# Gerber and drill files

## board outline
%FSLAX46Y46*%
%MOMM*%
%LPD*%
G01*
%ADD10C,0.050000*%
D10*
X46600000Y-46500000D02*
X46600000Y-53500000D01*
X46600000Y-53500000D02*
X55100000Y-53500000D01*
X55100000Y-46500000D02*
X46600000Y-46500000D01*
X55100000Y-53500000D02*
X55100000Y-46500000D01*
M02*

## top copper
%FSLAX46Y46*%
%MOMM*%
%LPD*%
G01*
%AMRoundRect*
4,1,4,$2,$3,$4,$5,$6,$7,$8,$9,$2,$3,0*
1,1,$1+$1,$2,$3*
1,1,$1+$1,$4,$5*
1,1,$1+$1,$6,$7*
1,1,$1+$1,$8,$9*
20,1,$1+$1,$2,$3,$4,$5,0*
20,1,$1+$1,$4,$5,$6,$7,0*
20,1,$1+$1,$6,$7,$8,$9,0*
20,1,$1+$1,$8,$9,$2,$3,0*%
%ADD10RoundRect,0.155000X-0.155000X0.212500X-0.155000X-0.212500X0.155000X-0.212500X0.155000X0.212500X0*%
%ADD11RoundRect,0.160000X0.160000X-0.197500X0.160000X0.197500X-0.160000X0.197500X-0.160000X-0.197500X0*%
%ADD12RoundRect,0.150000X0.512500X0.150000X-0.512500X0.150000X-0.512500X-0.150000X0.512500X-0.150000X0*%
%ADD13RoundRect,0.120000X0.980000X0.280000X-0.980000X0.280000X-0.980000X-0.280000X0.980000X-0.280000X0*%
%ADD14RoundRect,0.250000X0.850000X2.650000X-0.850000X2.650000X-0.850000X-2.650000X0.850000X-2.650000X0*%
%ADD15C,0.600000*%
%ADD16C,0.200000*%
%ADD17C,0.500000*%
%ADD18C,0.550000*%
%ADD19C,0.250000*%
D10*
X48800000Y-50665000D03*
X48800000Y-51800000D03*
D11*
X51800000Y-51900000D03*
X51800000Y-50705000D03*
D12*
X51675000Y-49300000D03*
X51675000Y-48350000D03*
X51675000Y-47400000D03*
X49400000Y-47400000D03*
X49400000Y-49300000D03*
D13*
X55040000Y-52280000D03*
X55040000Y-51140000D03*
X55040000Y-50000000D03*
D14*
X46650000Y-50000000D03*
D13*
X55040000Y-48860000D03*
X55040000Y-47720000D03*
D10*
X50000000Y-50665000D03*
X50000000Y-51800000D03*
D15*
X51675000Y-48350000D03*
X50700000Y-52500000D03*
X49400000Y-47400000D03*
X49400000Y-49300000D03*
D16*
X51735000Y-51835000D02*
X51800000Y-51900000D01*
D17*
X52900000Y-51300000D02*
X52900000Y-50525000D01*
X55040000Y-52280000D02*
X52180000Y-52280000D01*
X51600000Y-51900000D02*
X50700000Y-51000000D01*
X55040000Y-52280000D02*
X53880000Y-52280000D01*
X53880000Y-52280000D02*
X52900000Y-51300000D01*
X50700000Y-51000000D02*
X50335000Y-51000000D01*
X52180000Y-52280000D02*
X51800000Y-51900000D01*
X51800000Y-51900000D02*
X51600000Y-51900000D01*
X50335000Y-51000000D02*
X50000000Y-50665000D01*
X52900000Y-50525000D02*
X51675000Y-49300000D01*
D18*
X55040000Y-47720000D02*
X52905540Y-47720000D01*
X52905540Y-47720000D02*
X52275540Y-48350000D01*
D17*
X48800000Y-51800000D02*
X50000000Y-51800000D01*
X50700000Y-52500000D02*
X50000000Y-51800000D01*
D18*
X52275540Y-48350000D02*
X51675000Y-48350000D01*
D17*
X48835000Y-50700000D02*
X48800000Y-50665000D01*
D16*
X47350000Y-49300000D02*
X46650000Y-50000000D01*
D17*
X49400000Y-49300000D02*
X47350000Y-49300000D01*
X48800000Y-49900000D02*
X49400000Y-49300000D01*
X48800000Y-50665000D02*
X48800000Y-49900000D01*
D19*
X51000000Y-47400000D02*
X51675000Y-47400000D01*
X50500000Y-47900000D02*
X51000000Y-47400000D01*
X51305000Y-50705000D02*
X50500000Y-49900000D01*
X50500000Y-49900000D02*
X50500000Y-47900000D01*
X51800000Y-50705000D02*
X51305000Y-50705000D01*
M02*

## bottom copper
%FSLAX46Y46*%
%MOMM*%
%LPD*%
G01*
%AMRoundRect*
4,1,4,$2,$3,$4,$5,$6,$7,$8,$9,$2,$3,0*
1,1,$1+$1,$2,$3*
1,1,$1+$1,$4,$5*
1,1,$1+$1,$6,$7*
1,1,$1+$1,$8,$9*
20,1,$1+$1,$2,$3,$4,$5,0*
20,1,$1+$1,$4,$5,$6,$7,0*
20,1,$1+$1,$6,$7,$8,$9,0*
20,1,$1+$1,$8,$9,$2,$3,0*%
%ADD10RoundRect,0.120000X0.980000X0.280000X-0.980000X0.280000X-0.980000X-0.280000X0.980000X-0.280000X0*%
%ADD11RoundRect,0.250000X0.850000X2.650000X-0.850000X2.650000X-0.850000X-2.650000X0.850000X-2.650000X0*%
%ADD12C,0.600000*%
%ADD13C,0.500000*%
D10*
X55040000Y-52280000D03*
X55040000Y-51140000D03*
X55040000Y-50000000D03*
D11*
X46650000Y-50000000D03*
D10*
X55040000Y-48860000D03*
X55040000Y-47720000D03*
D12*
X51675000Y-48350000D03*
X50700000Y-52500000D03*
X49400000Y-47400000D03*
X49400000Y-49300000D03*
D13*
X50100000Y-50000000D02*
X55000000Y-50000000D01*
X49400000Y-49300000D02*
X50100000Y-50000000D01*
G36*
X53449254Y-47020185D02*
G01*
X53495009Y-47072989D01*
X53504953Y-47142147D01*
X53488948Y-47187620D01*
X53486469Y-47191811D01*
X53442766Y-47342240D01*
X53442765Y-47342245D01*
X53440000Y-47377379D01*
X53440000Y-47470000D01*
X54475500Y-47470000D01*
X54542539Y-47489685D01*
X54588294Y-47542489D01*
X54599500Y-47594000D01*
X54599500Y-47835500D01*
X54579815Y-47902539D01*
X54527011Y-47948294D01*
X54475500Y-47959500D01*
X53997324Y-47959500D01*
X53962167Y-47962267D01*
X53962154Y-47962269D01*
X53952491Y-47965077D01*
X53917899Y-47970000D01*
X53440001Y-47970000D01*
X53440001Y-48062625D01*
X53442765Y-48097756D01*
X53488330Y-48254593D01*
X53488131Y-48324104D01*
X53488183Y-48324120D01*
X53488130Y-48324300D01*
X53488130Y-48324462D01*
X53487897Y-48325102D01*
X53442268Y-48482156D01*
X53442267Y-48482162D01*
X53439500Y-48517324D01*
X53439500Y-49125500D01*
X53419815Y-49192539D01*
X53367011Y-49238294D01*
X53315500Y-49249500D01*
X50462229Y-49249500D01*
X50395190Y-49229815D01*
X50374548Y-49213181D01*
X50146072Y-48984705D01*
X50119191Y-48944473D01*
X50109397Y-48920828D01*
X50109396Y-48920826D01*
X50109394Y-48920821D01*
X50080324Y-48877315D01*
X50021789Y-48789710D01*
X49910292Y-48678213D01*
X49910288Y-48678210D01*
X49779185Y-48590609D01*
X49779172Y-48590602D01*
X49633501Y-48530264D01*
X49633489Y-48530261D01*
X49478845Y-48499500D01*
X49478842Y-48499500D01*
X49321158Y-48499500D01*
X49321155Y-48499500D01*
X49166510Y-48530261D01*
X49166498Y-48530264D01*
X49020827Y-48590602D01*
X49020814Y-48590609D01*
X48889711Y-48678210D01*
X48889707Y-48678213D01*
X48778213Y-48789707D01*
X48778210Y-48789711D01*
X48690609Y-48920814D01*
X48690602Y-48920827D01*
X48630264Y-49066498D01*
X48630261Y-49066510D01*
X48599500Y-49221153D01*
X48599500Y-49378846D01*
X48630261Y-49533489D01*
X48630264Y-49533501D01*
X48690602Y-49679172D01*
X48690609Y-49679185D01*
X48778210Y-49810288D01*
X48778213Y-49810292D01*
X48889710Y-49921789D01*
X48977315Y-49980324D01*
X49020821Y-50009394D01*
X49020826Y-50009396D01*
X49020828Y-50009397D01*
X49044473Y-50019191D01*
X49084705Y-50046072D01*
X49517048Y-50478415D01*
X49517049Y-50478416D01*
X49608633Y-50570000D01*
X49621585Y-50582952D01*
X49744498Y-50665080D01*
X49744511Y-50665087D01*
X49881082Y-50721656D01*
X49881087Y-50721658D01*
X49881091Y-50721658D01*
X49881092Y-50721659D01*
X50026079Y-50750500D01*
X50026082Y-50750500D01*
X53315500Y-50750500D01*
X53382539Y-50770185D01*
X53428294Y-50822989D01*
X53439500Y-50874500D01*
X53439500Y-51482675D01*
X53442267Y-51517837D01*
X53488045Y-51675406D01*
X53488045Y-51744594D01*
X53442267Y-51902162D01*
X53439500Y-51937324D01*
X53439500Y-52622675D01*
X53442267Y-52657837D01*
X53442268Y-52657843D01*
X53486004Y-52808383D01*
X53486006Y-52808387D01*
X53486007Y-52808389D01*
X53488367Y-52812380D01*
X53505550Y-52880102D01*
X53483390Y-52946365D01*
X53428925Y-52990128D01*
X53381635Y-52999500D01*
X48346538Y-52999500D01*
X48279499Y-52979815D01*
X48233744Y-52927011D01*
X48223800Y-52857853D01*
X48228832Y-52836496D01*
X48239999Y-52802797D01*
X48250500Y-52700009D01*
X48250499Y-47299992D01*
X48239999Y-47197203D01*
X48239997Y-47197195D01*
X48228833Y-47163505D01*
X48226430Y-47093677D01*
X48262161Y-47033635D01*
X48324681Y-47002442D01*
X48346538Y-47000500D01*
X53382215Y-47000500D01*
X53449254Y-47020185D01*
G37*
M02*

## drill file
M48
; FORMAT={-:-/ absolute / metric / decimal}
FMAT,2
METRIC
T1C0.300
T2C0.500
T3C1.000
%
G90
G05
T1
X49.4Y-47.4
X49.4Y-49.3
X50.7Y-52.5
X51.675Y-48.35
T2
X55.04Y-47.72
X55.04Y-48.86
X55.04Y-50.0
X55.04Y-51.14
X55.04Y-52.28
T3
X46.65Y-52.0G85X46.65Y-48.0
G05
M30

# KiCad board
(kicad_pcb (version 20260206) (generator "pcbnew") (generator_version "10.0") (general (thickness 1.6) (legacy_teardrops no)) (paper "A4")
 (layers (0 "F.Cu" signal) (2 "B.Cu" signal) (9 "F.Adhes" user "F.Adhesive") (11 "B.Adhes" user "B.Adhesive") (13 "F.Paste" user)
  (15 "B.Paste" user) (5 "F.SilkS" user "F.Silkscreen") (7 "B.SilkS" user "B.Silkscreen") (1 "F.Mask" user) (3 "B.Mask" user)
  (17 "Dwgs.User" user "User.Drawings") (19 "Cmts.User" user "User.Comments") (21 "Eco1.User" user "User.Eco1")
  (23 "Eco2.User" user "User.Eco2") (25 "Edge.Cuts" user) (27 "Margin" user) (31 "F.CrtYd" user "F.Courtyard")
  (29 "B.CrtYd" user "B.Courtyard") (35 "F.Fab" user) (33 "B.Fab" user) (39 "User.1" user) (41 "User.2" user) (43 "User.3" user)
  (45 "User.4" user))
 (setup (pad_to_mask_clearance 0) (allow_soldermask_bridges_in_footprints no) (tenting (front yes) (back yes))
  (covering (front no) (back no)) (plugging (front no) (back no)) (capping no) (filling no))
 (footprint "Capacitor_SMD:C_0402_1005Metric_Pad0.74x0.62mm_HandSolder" (layer "F.Cu") (at 48.8 51.2325 -90)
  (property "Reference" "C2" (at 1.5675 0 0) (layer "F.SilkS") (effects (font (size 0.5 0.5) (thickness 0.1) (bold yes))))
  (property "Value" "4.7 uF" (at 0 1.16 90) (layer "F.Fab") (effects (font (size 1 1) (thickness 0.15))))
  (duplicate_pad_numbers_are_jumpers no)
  (pad "1" smd roundrect (at -0.5675 0 270) (size 0.735 0.62) (layers "F.Cu" "F.Mask" "F.Paste") (roundrect_rratio 0.25) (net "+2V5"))
  (pad "2" smd roundrect (at 0.5675 0 270) (size 0.735 0.62) (layers "F.Cu" "F.Mask" "F.Paste") (roundrect_rratio 0.25) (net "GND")))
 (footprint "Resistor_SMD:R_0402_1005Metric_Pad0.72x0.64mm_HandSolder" (layer "F.Cu") (at 51.8 51.3025 90)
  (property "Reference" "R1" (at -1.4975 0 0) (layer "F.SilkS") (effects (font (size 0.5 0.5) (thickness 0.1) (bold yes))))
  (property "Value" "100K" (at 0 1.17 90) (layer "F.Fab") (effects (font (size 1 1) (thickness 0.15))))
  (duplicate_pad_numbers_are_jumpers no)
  (pad "1" smd roundrect (at -0.5975 0 90) (size 0.715 0.64) (layers "F.Cu" "F.Mask" "F.Paste") (roundrect_rratio 0.25) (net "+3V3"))
  (pad "2" smd roundrect (at 0.5975 0 90) (size 0.715 0.64) (layers "F.Cu" "F.Mask" "F.Paste") (roundrect_rratio 0.25) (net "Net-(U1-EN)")))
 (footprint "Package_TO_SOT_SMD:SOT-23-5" (layer "F.Cu") (at 50.5375 48.35 180)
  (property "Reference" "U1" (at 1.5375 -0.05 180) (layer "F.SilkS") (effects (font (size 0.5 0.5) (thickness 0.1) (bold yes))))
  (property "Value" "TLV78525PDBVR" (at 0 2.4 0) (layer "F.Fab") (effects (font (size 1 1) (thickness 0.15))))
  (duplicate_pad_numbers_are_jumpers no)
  (pad "1" smd roundrect (at -1.1375 -0.95 180) (size 1.325 0.6) (layers "F.Cu" "F.Mask" "F.Paste") (roundrect_rratio 0.25) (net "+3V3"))
  (pad "2" smd roundrect (at -1.1375 0 180) (size 1.325 0.6) (layers "F.Cu" "F.Mask" "F.Paste") (roundrect_rratio 0.25) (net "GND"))
  (pad "3" smd roundrect (at -1.1375 0.95 180) (size 1.325 0.6) (layers "F.Cu" "F.Mask" "F.Paste") (roundrect_rratio 0.25)
   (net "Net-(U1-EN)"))
  (pad "4" smd roundrect (at 1.1375 0.95 180) (size 1.325 0.6) (layers "F.Cu" "F.Mask" "F.Paste") (roundrect_rratio 0.25) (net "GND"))
  (pad "5" smd roundrect (at 1.1375 -0.95 180) (size 1.325 0.6) (layers "F.Cu" "F.Mask" "F.Paste") (roundrect_rratio 0.25) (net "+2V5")))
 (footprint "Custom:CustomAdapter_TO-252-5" (layer "F.Cu") (at 50 50 180)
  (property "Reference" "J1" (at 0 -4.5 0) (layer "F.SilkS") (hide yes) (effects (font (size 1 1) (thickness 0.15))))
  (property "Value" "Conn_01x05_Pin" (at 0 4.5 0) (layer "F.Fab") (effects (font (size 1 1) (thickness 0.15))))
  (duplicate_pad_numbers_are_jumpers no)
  (pad "1" thru_hole roundrect (at -5.04 -2.28 180) (size 2.2 0.8) (drill 0.5) (layers "*.Cu" "*.Mask") (remove_unused_layers no)
   (roundrect_rratio 0.15) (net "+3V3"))
  (pad "2" thru_hole roundrect (at -5.04 -1.14 180) (size 2.2 0.8) (drill 0.5) (layers "*.Cu" "*.Mask") (remove_unused_layers no)
   (roundrect_rratio 0.15) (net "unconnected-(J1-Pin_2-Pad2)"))
  (pad "3" thru_hole roundrect (at -5.04 0 180) (size 2.2 0.8) (drill 0.5) (layers "*.Cu" "*.Mask") (remove_unused_layers no)
   (roundrect_rratio 0.15) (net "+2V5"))
  (pad "3" thru_hole roundrect (at 3.35 0 180) (size 2.2 5.8) (drill oval 1 5) (layers "*.Cu" "*.Mask") (remove_unused_layers no)
   (roundrect_rratio 0.1136363636) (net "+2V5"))
  (pad "4" thru_hole roundrect (at -5.04 1.14 180) (size 2.2 0.8) (drill 0.5) (layers "*.Cu" "*.Mask") (remove_unused_layers no)
   (roundrect_rratio 0.15) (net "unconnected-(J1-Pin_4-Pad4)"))
  (pad "5" thru_hole roundrect (at -5.04 2.28 180) (size 2.2 0.8) (drill 0.5) (layers "*.Cu" "*.Mask") (remove_unused_layers no)
   (roundrect_rratio 0.15) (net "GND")))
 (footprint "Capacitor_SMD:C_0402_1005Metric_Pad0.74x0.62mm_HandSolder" (layer "F.Cu") (at 50 51.2325 -90)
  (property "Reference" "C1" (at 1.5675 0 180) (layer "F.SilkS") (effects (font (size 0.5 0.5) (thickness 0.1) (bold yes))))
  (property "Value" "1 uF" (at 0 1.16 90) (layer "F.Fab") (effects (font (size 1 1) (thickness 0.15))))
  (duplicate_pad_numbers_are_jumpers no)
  (pad "1" smd roundrect (at -0.5675 0 270) (size 0.735 0.62) (layers "F.Cu" "F.Mask" "F.Paste") (roundrect_rratio 0.25) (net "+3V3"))
  (pad "2" smd roundrect (at 0.5675 0 270) (size 0.735 0.62) (layers "F.Cu" "F.Mask" "F.Paste") (roundrect_rratio 0.25) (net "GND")))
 (gr_line (start 46.6 46.5) (end 46.6 53.5) (stroke (width 0.05) (type default)) (layer "Edge.Cuts"))
 (gr_line (start 46.6 53.5) (end 55.1 53.5) (stroke (width 0.05) (type default)) (layer "Edge.Cuts"))
 (gr_line (start 55.1 46.5) (end 46.6 46.5) (stroke (width 0.05) (type default)) (layer "Edge.Cuts"))
 (gr_line (start 55.1 53.5) (end 55.1 46.5) (stroke (width 0.05) (type default)) (layer "Edge.Cuts"))
 (segment (start 51.735 51.835) (end 51.8 51.9) (width 0.2) (layer "F.Cu") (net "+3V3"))
 (segment (start 52.9 51.3) (end 52.9 50.525) (width 0.5) (layer "F.Cu") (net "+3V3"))
 (segment (start 55.04 52.28) (end 52.18 52.28) (width 0.5) (layer "F.Cu") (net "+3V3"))
 (segment (start 51.6 51.9) (end 50.7 51) (width 0.5) (layer "F.Cu") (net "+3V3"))
 (segment (start 55.04 52.28) (end 53.88 52.28) (width 0.5) (layer "F.Cu") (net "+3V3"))
 (segment (start 53.88 52.28) (end 52.9 51.3) (width 0.5) (layer "F.Cu") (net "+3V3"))
 (segment (start 50.7 51) (end 50.335 51) (width 0.5) (layer "F.Cu") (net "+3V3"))
 (segment (start 52.18 52.28) (end 51.8 51.9) (width 0.5) (layer "F.Cu") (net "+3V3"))
 (segment (start 51.8 51.9) (end 51.6 51.9) (width 0.5) (layer "F.Cu") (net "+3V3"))
 (segment (start 50.335 51) (end 50 50.665) (width 0.5) (layer "F.Cu") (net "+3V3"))
 (segment (start 52.9 50.525) (end 51.675 49.3) (width 0.5) (layer "F.Cu") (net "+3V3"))
 (segment (start 55.04 47.72) (end 52.90554 47.72) (width 0.55) (layer "F.Cu") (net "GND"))
 (segment (start 52.90554 47.72) (end 52.27554 48.35) (width 0.55) (layer "F.Cu") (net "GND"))
 (segment (start 48.8 51.8) (end 50 51.8) (width 0.5) (layer "F.Cu") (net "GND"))
 (segment (start 50.7 52.5) (end 50 51.8) (width 0.5) (layer "F.Cu") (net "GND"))
 (segment (start 52.27554 48.35) (end 51.675 48.35) (width 0.55) (layer "F.Cu") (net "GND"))
 (via (at 51.675 48.35) (size 0.6) (drill 0.3) (layers "F.Cu" "B.Cu") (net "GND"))
 (via (at 50.7 52.5) (size 0.6) (drill 0.3) (layers "F.Cu" "B.Cu") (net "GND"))
 (via (at 49.4 47.4) (size 0.6) (drill 0.3) (layers "F.Cu" "B.Cu") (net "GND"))
 (segment (start 48.835 50.7) (end 48.8 50.665) (width 0.5) (layer "F.Cu") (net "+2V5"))
 (segment (start 47.35 49.3) (end 46.65 50) (width 0.2) (layer "F.Cu") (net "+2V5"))
 (segment (start 49.4 49.3) (end 47.35 49.3) (width 0.5) (layer "F.Cu") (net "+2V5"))
 (segment (start 48.8 49.9) (end 49.4 49.3) (width 0.5) (layer "F.Cu") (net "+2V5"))
 (segment (start 48.8 50.665) (end 48.8 49.9) (width 0.5) (layer "F.Cu") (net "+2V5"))
 (via (at 49.4 49.3) (size 0.6) (drill 0.3) (layers "F.Cu" "B.Cu") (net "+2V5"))
 (segment (start 50.1 50) (end 55 50) (width 0.5) (layer "B.Cu") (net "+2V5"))
 (segment (start 49.4 49.3) (end 50.1 50) (width 0.5) (layer "B.Cu") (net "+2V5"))
 (segment (start 51 47.4) (end 51.675 47.4) (width 0.25) (layer "F.Cu") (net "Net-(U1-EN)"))
 (segment (start 50.5 47.9) (end 51 47.4) (width 0.25) (layer "F.Cu") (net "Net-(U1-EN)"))
 (segment (start 51.305 50.705) (end 50.5 49.9) (width 0.25) (layer "F.Cu") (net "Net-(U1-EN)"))
 (segment (start 50.5 49.9) (end 50.5 47.9) (width 0.25) (layer "F.Cu") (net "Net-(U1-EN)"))
 (segment (start 51.8 50.705) (end 51.305 50.705) (width 0.25) (layer "F.Cu") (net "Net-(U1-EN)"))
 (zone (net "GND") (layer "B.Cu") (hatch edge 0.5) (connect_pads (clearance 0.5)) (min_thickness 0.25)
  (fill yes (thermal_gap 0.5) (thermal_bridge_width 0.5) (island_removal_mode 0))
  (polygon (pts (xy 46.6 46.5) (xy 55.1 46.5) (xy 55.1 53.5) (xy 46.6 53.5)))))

